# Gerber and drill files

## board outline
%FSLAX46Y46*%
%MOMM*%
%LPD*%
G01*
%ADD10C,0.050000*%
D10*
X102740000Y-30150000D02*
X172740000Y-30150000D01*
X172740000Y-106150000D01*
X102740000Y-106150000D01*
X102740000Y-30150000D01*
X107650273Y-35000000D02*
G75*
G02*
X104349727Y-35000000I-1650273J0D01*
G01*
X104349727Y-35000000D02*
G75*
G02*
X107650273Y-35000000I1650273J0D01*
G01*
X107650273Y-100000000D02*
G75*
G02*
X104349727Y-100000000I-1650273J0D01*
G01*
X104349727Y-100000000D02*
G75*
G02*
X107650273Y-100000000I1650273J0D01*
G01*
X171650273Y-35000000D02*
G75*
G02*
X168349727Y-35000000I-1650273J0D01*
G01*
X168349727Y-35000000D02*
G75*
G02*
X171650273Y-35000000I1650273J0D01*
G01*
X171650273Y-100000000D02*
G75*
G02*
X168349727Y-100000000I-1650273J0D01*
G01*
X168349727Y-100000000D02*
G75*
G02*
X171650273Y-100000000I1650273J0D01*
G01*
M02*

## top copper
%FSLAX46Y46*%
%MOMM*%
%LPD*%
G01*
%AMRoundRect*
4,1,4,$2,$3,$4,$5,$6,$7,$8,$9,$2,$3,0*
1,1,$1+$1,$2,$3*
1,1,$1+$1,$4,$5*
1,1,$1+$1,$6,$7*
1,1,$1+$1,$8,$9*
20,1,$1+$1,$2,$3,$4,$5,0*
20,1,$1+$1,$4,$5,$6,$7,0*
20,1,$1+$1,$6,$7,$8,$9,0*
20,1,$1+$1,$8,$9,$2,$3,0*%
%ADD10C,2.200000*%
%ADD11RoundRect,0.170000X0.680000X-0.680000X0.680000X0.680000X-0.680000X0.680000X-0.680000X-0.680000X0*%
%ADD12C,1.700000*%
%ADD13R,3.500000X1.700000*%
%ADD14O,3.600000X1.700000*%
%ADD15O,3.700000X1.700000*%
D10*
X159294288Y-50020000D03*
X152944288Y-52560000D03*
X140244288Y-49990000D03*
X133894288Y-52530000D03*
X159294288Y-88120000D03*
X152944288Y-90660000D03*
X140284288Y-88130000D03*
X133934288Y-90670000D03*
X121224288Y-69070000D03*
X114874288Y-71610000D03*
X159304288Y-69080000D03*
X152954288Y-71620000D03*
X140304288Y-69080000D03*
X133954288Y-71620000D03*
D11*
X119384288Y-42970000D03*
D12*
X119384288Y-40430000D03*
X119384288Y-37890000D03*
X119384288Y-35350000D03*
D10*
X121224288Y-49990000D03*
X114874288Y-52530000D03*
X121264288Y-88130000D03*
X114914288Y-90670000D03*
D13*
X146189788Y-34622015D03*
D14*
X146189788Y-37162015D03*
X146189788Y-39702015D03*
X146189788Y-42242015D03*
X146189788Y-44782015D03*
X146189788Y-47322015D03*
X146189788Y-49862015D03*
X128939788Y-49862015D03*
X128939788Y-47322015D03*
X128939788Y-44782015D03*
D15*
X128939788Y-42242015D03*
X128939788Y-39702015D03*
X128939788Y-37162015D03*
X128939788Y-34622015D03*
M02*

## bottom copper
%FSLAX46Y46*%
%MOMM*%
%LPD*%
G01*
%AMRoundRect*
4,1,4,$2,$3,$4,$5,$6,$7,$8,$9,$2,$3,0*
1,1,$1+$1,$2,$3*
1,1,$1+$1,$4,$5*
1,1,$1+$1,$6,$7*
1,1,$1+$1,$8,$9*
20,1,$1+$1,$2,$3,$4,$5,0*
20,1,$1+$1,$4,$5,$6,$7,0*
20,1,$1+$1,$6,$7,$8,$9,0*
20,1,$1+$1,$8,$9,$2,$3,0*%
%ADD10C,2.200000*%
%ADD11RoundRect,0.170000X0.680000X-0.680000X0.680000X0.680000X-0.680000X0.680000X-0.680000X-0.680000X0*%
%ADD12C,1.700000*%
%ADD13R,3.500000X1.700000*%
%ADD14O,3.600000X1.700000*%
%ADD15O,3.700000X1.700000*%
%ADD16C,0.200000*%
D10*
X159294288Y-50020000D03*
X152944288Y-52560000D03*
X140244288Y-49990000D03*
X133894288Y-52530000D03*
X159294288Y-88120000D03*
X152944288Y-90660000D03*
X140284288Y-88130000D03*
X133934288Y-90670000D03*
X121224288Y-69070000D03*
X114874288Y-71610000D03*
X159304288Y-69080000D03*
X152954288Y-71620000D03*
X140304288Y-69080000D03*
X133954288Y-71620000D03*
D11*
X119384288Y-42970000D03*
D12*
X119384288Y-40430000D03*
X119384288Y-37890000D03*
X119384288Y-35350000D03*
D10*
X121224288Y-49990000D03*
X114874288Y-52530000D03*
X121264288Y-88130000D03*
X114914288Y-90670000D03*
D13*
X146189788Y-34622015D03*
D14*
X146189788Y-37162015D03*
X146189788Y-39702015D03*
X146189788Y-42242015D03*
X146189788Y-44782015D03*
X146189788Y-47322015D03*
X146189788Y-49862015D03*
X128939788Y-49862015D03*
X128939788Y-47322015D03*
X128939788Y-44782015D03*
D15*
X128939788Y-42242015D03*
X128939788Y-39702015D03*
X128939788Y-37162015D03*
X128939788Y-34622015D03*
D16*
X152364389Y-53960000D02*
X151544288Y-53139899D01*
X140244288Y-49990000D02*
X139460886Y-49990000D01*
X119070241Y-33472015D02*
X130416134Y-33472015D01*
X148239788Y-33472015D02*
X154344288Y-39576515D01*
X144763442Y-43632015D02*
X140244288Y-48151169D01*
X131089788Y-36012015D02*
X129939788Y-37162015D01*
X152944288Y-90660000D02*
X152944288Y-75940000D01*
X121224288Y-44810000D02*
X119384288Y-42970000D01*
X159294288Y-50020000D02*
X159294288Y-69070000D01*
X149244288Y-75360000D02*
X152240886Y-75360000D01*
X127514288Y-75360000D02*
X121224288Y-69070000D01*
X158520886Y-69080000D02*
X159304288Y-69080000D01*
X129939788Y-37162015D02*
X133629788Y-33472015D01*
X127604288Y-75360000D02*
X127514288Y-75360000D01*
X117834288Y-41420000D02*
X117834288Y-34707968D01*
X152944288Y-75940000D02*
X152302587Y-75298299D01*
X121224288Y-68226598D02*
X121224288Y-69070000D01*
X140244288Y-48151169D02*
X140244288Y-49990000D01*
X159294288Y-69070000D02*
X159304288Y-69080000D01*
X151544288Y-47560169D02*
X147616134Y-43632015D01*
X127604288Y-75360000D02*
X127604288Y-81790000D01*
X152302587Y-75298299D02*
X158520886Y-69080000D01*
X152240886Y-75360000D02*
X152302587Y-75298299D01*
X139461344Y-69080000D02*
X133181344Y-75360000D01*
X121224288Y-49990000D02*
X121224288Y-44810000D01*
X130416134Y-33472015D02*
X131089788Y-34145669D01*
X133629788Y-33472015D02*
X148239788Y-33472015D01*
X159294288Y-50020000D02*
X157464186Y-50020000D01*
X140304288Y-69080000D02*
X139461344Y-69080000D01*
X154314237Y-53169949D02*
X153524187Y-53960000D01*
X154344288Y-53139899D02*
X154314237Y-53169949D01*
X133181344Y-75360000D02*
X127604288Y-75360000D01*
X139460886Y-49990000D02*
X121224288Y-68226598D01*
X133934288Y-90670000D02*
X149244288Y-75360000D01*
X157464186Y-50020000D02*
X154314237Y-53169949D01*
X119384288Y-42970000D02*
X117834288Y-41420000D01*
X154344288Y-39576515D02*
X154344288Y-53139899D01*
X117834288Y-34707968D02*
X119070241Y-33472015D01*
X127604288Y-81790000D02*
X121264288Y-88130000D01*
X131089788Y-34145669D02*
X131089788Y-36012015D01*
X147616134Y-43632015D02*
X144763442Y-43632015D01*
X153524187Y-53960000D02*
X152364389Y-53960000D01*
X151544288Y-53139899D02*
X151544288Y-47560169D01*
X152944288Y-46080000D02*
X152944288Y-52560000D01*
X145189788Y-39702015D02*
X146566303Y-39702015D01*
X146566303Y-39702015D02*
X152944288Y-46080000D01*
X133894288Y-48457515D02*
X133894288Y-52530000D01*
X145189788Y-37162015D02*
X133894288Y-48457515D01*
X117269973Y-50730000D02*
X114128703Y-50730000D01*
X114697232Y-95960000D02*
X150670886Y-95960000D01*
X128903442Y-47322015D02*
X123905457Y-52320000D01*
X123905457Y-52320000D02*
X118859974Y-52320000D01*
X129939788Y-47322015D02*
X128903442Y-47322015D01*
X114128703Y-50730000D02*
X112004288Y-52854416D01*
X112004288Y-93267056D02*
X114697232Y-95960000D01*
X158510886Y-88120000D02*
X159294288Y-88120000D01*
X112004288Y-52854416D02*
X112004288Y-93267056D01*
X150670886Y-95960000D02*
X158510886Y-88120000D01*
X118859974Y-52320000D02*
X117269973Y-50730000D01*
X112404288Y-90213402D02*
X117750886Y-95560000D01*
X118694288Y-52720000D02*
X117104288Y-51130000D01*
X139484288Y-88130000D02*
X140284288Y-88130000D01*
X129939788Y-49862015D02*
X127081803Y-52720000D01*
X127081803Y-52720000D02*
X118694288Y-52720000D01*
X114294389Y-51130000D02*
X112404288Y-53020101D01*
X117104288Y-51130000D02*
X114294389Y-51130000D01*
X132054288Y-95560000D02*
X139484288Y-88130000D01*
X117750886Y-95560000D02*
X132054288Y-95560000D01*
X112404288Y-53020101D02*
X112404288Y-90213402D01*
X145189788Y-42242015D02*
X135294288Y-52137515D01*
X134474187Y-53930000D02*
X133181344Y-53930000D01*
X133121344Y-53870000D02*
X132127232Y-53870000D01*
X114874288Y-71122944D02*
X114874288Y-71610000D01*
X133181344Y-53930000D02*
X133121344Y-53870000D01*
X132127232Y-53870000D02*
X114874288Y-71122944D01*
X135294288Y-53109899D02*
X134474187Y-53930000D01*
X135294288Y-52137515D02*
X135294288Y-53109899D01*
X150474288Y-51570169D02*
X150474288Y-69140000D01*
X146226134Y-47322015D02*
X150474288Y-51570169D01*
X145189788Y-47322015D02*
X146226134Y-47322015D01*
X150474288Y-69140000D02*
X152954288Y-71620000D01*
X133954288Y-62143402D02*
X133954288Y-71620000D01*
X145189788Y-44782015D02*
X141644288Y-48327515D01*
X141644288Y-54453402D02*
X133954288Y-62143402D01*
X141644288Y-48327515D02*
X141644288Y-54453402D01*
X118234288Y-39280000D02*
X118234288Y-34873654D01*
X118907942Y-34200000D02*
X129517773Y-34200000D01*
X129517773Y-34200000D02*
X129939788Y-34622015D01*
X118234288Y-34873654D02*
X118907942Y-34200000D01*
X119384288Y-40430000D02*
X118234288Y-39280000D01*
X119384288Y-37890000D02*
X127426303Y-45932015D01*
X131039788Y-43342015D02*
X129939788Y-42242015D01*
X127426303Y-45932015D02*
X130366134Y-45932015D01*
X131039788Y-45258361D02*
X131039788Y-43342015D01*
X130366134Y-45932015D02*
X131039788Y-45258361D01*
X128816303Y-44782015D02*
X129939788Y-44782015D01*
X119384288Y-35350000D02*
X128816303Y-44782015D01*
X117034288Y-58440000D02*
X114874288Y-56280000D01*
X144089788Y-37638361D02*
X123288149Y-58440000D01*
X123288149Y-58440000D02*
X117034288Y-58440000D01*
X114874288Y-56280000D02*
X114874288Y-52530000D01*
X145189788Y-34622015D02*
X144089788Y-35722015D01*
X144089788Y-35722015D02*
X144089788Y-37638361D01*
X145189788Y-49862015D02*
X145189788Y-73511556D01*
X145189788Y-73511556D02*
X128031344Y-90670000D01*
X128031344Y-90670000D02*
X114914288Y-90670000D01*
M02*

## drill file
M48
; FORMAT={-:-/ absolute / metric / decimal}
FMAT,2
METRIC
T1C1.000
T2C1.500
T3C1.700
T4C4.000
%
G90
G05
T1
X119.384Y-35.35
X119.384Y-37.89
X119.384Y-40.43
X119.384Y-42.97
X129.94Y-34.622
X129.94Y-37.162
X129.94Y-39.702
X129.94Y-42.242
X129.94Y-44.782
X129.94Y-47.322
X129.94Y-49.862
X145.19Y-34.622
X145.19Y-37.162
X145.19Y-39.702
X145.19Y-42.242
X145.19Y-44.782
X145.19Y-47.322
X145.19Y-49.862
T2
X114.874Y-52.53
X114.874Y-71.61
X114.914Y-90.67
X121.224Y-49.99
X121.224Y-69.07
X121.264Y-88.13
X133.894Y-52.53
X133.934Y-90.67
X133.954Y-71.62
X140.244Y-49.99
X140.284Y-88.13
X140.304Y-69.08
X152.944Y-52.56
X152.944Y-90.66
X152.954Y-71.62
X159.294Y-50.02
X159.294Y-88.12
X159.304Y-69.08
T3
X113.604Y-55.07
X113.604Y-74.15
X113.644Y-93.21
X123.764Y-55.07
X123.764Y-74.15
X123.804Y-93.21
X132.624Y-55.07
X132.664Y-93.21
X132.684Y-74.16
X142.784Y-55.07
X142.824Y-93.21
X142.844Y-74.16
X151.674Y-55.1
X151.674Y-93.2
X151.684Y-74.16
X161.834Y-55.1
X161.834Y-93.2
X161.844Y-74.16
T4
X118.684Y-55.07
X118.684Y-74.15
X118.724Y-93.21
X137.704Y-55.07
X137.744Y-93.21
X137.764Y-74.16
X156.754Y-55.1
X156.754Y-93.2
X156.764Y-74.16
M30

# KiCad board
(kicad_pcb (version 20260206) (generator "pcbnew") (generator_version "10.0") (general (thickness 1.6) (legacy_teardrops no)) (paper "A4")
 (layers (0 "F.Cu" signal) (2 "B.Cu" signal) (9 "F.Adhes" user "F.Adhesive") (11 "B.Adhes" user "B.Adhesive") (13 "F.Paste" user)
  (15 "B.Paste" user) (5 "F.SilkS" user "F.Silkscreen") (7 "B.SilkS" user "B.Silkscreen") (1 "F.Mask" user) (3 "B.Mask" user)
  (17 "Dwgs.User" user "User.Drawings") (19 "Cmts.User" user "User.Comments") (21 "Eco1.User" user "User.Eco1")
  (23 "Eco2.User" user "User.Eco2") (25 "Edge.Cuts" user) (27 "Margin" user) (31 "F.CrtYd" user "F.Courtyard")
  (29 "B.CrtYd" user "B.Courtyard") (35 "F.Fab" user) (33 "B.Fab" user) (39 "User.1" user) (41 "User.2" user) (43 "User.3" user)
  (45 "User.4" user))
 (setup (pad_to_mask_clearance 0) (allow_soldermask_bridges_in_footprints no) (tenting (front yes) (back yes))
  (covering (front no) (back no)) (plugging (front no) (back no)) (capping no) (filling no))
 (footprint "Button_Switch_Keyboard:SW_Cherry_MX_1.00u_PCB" (layer "F.Cu") (at 159.294288 50.02)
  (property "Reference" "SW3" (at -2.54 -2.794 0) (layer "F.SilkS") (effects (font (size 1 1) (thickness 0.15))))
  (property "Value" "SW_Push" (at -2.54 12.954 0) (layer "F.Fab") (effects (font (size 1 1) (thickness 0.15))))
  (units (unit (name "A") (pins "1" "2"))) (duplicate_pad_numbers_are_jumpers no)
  (pad "" np_thru_hole circle (at -7.62 5.08) (size 1.7 1.7) (drill 1.7) (layers "*.Cu" "*.Mask"))
  (pad "" np_thru_hole circle (at -2.54 5.08) (size 4 4) (drill 4) (layers "*.Cu" "*.Mask"))
  (pad "" np_thru_hole circle (at 2.54 5.08) (size 1.7 1.7) (drill 1.7) (layers "*.Cu" "*.Mask"))
  (pad "1" thru_hole circle (at 0 0) (size 2.2 2.2) (drill 1.5) (layers "*.Cu" "*.Mask") (remove_unused_layers no) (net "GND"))
  (pad "2" thru_hole circle (at -6.35 2.54) (size 2.2 2.2) (drill 1.5) (layers "*.Cu" "*.Mask") (remove_unused_layers no)
   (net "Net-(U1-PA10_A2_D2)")))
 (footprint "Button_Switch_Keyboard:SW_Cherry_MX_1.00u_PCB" (layer "F.Cu") (at 140.244288 49.99)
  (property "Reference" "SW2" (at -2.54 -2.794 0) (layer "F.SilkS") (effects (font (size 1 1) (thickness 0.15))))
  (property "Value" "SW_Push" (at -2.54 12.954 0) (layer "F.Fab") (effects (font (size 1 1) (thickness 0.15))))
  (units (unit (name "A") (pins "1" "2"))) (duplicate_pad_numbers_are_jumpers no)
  (pad "" np_thru_hole circle (at -7.62 5.08) (size 1.7 1.7) (drill 1.7) (layers "*.Cu" "*.Mask"))
  (pad "" np_thru_hole circle (at -2.54 5.08) (size 4 4) (drill 4) (layers "*.Cu" "*.Mask"))
  (pad "" np_thru_hole circle (at 2.54 5.08) (size 1.7 1.7) (drill 1.7) (layers "*.Cu" "*.Mask"))
  (pad "1" thru_hole circle (at 0 0) (size 2.2 2.2) (drill 1.5) (layers "*.Cu" "*.Mask") (remove_unused_layers no) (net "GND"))
  (pad "2" thru_hole circle (at -6.35 2.54) (size 2.2 2.2) (drill 1.5) (layers "*.Cu" "*.Mask") (remove_unused_layers no)
   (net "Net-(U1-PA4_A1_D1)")))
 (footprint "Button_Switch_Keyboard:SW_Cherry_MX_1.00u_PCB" (layer "F.Cu") (at 159.294288 88.12)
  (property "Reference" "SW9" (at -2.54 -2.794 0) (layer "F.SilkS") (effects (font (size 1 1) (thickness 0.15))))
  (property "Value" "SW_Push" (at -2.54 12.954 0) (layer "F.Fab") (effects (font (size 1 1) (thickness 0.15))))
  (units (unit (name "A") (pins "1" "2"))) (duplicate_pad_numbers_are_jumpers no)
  (pad "" np_thru_hole circle (at -7.62 5.08) (size 1.7 1.7) (drill 1.7) (layers "*.Cu" "*.Mask"))
  (pad "" np_thru_hole circle (at -2.54 5.08) (size 4 4) (drill 4) (layers "*.Cu" "*.Mask"))
  (pad "" np_thru_hole circle (at 2.54 5.08) (size 1.7 1.7) (drill 1.7) (layers "*.Cu" "*.Mask"))
  (pad "1" thru_hole circle (at 0 0) (size 2.2 2.2) (drill 1.5) (layers "*.Cu" "*.Mask") (remove_unused_layers no)
   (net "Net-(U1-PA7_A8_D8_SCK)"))
  (pad "2" thru_hole circle (at -6.35 2.54) (size 2.2 2.2) (drill 1.5) (layers "*.Cu" "*.Mask") (remove_unused_layers no) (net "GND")))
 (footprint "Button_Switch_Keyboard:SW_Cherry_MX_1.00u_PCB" (layer "F.Cu") (at 140.284288 88.13)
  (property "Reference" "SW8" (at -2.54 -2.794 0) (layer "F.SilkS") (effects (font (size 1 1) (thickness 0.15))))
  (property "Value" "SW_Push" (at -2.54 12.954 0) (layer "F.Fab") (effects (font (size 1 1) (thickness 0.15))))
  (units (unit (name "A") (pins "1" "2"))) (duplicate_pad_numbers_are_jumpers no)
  (pad "" np_thru_hole circle (at -7.62 5.08) (size 1.7 1.7) (drill 1.7) (layers "*.Cu" "*.Mask"))
  (pad "" np_thru_hole circle (at -2.54 5.08) (size 4 4) (drill 4) (layers "*.Cu" "*.Mask"))
  (pad "" np_thru_hole circle (at 2.54 5.08) (size 1.7 1.7) (drill 1.7) (layers "*.Cu" "*.Mask"))
  (pad "1" thru_hole circle (at 0 0) (size 2.2 2.2) (drill 1.5) (layers "*.Cu" "*.Mask") (remove_unused_layers no)
   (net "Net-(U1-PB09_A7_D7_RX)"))
  (pad "2" thru_hole circle (at -6.35 2.54) (size 2.2 2.2) (drill 1.5) (layers "*.Cu" "*.Mask") (remove_unused_layers no) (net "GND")))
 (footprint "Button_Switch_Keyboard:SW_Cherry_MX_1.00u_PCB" (layer "F.Cu") (at 121.224288 69.07)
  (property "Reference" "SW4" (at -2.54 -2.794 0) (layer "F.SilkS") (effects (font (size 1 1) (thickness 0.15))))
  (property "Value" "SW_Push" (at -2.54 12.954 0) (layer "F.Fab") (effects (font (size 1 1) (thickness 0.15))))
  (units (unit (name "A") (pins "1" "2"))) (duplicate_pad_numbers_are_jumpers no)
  (pad "" np_thru_hole circle (at -7.62 5.08) (size 1.7 1.7) (drill 1.7) (layers "*.Cu" "*.Mask"))
  (pad "" np_thru_hole circle (at -2.54 5.08) (size 4 4) (drill 4) (layers "*.Cu" "*.Mask"))
  (pad "" np_thru_hole circle (at 2.54 5.08) (size 1.7 1.7) (drill 1.7) (layers "*.Cu" "*.Mask"))
  (pad "1" thru_hole circle (at 0 0) (size 2.2 2.2) (drill 1.5) (layers "*.Cu" "*.Mask") (remove_unused_layers no) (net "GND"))
  (pad "2" thru_hole circle (at -6.35 2.54) (size 2.2 2.2) (drill 1.5) (layers "*.Cu" "*.Mask") (remove_unused_layers no)
   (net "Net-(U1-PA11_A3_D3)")))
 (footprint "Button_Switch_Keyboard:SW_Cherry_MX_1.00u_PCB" (layer "F.Cu") (at 159.304288 69.08)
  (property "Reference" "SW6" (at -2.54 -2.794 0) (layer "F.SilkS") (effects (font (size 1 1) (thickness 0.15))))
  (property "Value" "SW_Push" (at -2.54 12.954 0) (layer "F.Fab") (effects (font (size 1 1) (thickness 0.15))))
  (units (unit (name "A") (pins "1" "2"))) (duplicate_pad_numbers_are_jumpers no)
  (pad "" np_thru_hole circle (at -7.62 5.08) (size 1.7 1.7) (drill 1.7) (layers "*.Cu" "*.Mask"))
  (pad "" np_thru_hole circle (at -2.54 5.08) (size 4 4) (drill 4) (layers "*.Cu" "*.Mask"))
  (pad "" np_thru_hole circle (at 2.54 5.08) (size 1.7 1.7) (drill 1.7) (layers "*.Cu" "*.Mask"))
  (pad "1" thru_hole circle (at 0 0) (size 2.2 2.2) (drill 1.5) (layers "*.Cu" "*.Mask") (remove_unused_layers no) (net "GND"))
  (pad "2" thru_hole circle (at -6.35 2.54) (size 2.2 2.2) (drill 1.5) (layers "*.Cu" "*.Mask") (remove_unused_layers no)
   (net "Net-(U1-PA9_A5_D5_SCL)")))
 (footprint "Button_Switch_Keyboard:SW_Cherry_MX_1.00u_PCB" (layer "F.Cu") (at 140.304288 69.08)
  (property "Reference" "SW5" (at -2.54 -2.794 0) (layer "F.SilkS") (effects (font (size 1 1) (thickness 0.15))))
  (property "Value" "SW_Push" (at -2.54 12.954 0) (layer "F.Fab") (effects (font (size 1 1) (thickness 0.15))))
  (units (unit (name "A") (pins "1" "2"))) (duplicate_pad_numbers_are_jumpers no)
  (pad "" np_thru_hole circle (at -7.62 5.08) (size 1.7 1.7) (drill 1.7) (layers "*.Cu" "*.Mask"))
  (pad "" np_thru_hole circle (at -2.54 5.08) (size 4 4) (drill 4) (layers "*.Cu" "*.Mask"))
  (pad "" np_thru_hole circle (at 2.54 5.08) (size 1.7 1.7) (drill 1.7) (layers "*.Cu" "*.Mask"))
  (pad "1" thru_hole circle (at 0 0) (size 2.2 2.2) (drill 1.5) (layers "*.Cu" "*.Mask") (remove_unused_layers no) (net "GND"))
  (pad "2" thru_hole circle (at -6.35 2.54) (size 2.2 2.2) (drill 1.5) (layers "*.Cu" "*.Mask") (remove_unused_layers no)
   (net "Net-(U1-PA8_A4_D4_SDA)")))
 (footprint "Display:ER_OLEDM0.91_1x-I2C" (layer "F.Cu") (at 119.384288 42.97 90)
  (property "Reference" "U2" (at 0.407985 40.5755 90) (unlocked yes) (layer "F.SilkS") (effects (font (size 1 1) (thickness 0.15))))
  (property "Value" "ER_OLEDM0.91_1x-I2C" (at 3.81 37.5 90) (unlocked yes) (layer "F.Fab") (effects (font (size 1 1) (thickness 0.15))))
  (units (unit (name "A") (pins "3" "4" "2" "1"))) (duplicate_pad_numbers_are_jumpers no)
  (pad "1" thru_hole roundrect (at 0 0 90) (size 1.7 1.7) (drill 1) (layers "*.Cu" "*.Mask") (remove_unused_layers no)
   (roundrect_rratio 0.1) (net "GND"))
  (pad "2" thru_hole circle (at 2.54 0 90) (size 1.7 1.7) (drill 1) (layers "*.Cu" "*.Mask") (remove_unused_layers no) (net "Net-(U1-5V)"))
  (pad "3" thru_hole circle (at 5.08 0 90) (size 1.7 1.7) (drill 1) (layers "*.Cu" "*.Mask") (remove_unused_layers no)
   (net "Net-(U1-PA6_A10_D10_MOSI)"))
  (pad "4" thru_hole circle (at 7.62 0 90) (size 1.7 1.7) (drill 1) (layers "*.Cu" "*.Mask") (remove_unused_layers no)
   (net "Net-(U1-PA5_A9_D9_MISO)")))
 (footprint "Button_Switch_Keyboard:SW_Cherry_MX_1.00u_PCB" (layer "F.Cu") (at 121.224288 49.99)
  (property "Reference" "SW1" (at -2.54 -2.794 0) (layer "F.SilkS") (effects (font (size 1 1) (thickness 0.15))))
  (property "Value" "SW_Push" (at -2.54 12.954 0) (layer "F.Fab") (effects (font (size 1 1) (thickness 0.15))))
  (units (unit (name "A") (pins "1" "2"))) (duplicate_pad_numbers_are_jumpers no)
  (pad "" np_thru_hole circle (at -7.62 5.08) (size 1.7 1.7) (drill 1.7) (layers "*.Cu" "*.Mask"))
  (pad "" np_thru_hole circle (at -2.54 5.08) (size 4 4) (drill 4) (layers "*.Cu" "*.Mask"))
  (pad "" np_thru_hole circle (at 2.54 5.08) (size 1.7 1.7) (drill 1.7) (layers "*.Cu" "*.Mask"))
  (pad "1" thru_hole circle (at 0 0) (size 2.2 2.2) (drill 1.5) (layers "*.Cu" "*.Mask") (remove_unused_layers no) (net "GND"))
  (pad "2" thru_hole circle (at -6.35 2.54) (size 2.2 2.2) (drill 1.5) (layers "*.Cu" "*.Mask") (remove_unused_layers no)
   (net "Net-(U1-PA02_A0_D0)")))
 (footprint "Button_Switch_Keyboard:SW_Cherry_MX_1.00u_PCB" (layer "F.Cu") (at 121.264288 88.13)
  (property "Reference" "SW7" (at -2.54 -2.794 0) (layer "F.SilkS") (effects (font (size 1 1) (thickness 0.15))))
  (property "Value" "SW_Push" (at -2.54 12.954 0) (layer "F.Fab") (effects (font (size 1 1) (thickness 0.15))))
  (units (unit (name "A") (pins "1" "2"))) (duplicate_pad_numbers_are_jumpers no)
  (pad "" np_thru_hole circle (at -7.62 5.08) (size 1.7 1.7) (drill 1.7) (layers "*.Cu" "*.Mask"))
  (pad "" np_thru_hole circle (at -2.54 5.08) (size 4 4) (drill 4) (layers "*.Cu" "*.Mask"))
  (pad "" np_thru_hole circle (at 2.54 5.08) (size 1.7 1.7) (drill 1.7) (layers "*.Cu" "*.Mask"))
  (pad "1" thru_hole circle (at 0 0) (size 2.2 2.2) (drill 1.5) (layers "*.Cu" "*.Mask") (remove_unused_layers no) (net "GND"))
  (pad "2" thru_hole circle (at -6.35 2.54) (size 2.2 2.2) (drill 1.5) (layers "*.Cu" "*.Mask") (remove_unused_layers no)
   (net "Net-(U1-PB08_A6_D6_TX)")))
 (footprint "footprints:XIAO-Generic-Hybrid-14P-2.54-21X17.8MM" (layer "B.Cu") (at 137.564788 42.242015 180)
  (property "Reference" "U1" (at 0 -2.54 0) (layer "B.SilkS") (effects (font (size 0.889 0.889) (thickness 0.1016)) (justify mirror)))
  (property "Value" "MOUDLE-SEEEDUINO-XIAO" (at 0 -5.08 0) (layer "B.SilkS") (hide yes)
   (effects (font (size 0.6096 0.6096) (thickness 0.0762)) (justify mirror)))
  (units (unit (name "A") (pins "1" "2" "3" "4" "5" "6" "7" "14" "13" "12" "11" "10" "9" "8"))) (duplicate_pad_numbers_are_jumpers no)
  (pad "1" thru_hole rect (at -7.625 7.62 180) (size 3.5 1.7) (drill 1 (offset -1 0)) (layers "*.Cu" "*.Mask") (remove_unused_layers no)
   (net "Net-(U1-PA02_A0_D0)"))
  (pad "2" thru_hole oval (at -7.625 5.08 180) (size 3.6 1.7) (drill 1 (offset -1 0)) (layers "*.Cu" "*.Mask") (remove_unused_layers no)
   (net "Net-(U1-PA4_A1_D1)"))
  (pad "3" thru_hole oval (at -7.625 2.54 180) (size 3.6 1.7) (drill 1 (offset -1 0)) (layers "*.Cu" "*.Mask") (remove_unused_layers no)
   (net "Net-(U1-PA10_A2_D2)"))
  (pad "4" thru_hole oval (at -7.625 0 180) (size 3.6 1.7) (drill 1 (offset -1 0)) (layers "*.Cu" "*.Mask") (remove_unused_layers no)
   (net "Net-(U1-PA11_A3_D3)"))
  (pad "5" thru_hole oval (at -7.625 -2.54 180) (size 3.6 1.7) (drill 1 (offset -1 0)) (layers "*.Cu" "*.Mask") (remove_unused_layers no)
   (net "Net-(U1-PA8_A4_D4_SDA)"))
  (pad "6" thru_hole oval (at -7.625 -5.08) (size 3.6 1.7) (drill 1 (offset 1 0)) (layers "*.Cu" "*.Mask") (remove_unused_layers no)
   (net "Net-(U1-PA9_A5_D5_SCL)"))
  (pad "7" thru_hole oval (at -7.625 -7.62 180) (size 3.6 1.7) (drill 1 (offset -1 0)) (layers "*.Cu" "*.Mask") (remove_unused_layers no)
   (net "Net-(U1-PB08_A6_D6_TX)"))
  (pad "8" thru_hole oval (at 7.625 -7.62 180) (size 3.6 1.7) (drill 1 (offset 1 0)) (layers "*.Cu" "*.Mask") (remove_unused_layers no)
   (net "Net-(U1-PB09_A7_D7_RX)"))
  (pad "9" thru_hole oval (at 7.625 -5.08 180) (size 3.6 1.7) (drill 1 (offset 1 0)) (layers "*.Cu" "*.Mask") (remove_unused_layers no)
   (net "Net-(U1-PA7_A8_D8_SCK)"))
  (pad "10" thru_hole oval (at 7.625 -2.54 180) (size 3.6 1.7) (drill 1 (offset 1 0)) (layers "*.Cu" "*.Mask") (remove_unused_layers no)
   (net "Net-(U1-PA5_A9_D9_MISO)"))
  (pad "11" thru_hole oval (at 7.625 0 180) (size 3.7 1.7) (drill 1 (offset 1 0)) (layers "*.Cu" "*.Mask") (remove_unused_layers no)
   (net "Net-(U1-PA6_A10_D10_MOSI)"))
  (pad "12" thru_hole oval (at 7.625 2.54 180) (size 3.7 1.7) (drill 1 (offset 1 0)) (layers "*.Cu" "*.Mask") (remove_unused_layers no)
   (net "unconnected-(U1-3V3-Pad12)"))
  (pad "13" thru_hole oval (at 7.625 5.08 180) (size 3.7 1.7) (drill 1 (offset 1 0)) (layers "*.Cu" "*.Mask") (remove_unused_layers no)
   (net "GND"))
  (pad "14" thru_hole oval (at 7.625 7.62 180) (size 3.7 1.7) (drill 1 (offset 1 0)) (layers "*.Cu" "*.Mask") (remove_unused_layers no)
   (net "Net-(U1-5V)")))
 (gr_rect (start 102.74 30.15) (end 172.74 106.15) (stroke (width 0.05) (type solid)) (fill no) (layer "Edge.Cuts"))
 (gr_circle (center 106 35) (end 107.650273 35) (stroke (width 0.05) (type solid)) (fill no) (layer "Edge.Cuts"))
 (gr_circle (center 106 100) (end 107.650273 100) (stroke (width 0.05) (type solid)) (fill no) (layer "Edge.Cuts"))
 (gr_circle (center 170 35) (end 171.650273 35) (stroke (width 0.05) (type solid)) (fill no) (layer "Edge.Cuts"))
 (gr_circle (center 170 100) (end 171.650273 100) (stroke (width 0.05) (type solid)) (fill no) (layer "Edge.Cuts"))
 (segment (start 152.364389 53.96) (end 151.544288 53.139899) (width 0.2) (layer "B.Cu") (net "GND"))
 (segment (start 140.244288 49.99) (end 139.460886 49.99) (width 0.2) (layer "B.Cu") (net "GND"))
 (segment (start 119.070241 33.472015) (end 130.416134 33.472015) (width 0.2) (layer "B.Cu") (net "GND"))
 (segment (start 148.239788 33.472015) (end 154.344288 39.576515) (width 0.2) (layer "B.Cu") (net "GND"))
 (segment (start 144.763442 43.632015) (end 140.244288 48.151169) (width 0.2) (layer "B.Cu") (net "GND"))
 (segment (start 131.089788 36.012015) (end 129.939788 37.162015) (width 0.2) (layer "B.Cu") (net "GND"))
 (segment (start 152.944288 90.66) (end 152.944288 75.94) (width 0.2) (layer "B.Cu") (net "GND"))
 (segment (start 121.224288 44.81) (end 119.384288 42.97) (width 0.2) (layer "B.Cu") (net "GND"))
 (segment (start 159.294288 50.02) (end 159.294288 69.07) (width 0.2) (layer "B.Cu") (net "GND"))
 (segment (start 149.244288 75.36) (end 152.240886 75.36) (width 0.2) (layer "B.Cu") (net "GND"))
 (segment (start 127.514288 75.36) (end 121.224288 69.07) (width 0.2) (layer "B.Cu") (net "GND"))
 (segment (start 158.520886 69.08) (end 159.304288 69.08) (width 0.2) (layer "B.Cu") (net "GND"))
 (segment (start 129.939788 37.162015) (end 133.629788 33.472015) (width 0.2) (layer "B.Cu") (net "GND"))
 (segment (start 127.604288 75.36) (end 127.514288 75.36) (width 0.2) (layer "B.Cu") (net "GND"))
 (segment (start 117.834288 41.42) (end 117.834288 34.707968) (width 0.2) (layer "B.Cu") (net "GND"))
 (segment (start 152.944288 75.94) (end 152.302587 75.298299) (width 0.2) (layer "B.Cu") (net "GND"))
 (segment (start 121.224288 68.226598) (end 121.224288 69.07) (width 0.2) (layer "B.Cu") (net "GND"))
 (segment (start 140.244288 48.151169) (end 140.244288 49.99) (width 0.2) (layer "B.Cu") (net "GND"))
 (segment (start 159.294288 69.07) (end 159.304288 69.08) (width 0.2) (layer "B.Cu") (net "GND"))
 (segment (start 151.544288 47.560169) (end 147.616134 43.632015) (width 0.2) (layer "B.Cu") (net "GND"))
 (segment (start 127.604288 75.36) (end 127.604288 81.79) (width 0.2) (layer "B.Cu") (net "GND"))
 (segment (start 152.302587 75.298299) (end 158.520886 69.08) (width 0.2) (layer "B.Cu") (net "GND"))
 (segment (start 152.240886 75.36) (end 152.302587 75.298299) (width 0.2) (layer "B.Cu") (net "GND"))
 (segment (start 139.461344 69.08) (end 133.181344 75.36) (width 0.2) (layer "B.Cu") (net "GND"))
 (segment (start 121.224288 49.99) (end 121.224288 44.81) (width 0.2) (layer "B.Cu") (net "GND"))
 (segment (start 130.416134 33.472015) (end 131.089788 34.145669) (width 0.2) (layer "B.Cu") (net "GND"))
 (segment (start 133.629788 33.472015) (end 148.239788 33.472015) (width 0.2) (layer "B.Cu") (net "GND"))
 (segment (start 159.294288 50.02) (end 157.464186 50.02) (width 0.2) (layer "B.Cu") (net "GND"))
 (segment (start 140.304288 69.08) (end 139.461344 69.08) (width 0.2) (layer "B.Cu") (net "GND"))
 (segment (start 154.314237 53.169949) (end 153.524187 53.96) (width 0.2) (layer "B.Cu") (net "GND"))
 (segment (start 154.344288 53.139899) (end 154.314237 53.169949) (width 0.2) (layer "B.Cu") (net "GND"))
 (segment (start 133.181344 75.36) (end 127.604288 75.36) (width 0.2) (layer "B.Cu") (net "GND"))
 (segment (start 139.460886 49.99) (end 121.224288 68.226598) (width 0.2) (layer "B.Cu") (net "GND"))
 (segment (start 133.934288 90.67) (end 149.244288 75.36) (width 0.2) (layer "B.Cu") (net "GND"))
 (segment (start 157.464186 50.02) (end 154.314237 53.169949) (width 0.2) (layer "B.Cu") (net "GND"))
 (segment (start 119.384288 42.97) (end 117.834288 41.42) (width 0.2) (layer "B.Cu") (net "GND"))
 (segment (start 154.344288 39.576515) (end 154.344288 53.139899) (width 0.2) (layer "B.Cu") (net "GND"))
 (segment (start 117.834288 34.707968) (end 119.070241 33.472015) (width 0.2) (layer "B.Cu") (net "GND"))
 (segment (start 127.604288 81.79) (end 121.264288 88.13) (width 0.2) (layer "B.Cu") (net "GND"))
 (segment (start 131.089788 34.145669) (end 131.089788 36.012015) (width 0.2) (layer "B.Cu") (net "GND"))
 (segment (start 147.616134 43.632015) (end 144.763442 43.632015) (width 0.2) (layer "B.Cu") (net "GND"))
 (segment (start 153.524187 53.96) (end 152.364389 53.96) (width 0.2) (layer "B.Cu") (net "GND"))
 (segment (start 151.544288 53.139899) (end 151.544288 47.560169) (width 0.2) (layer "B.Cu") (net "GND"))
 (segment (start 152.944288 46.08) (end 152.944288 52.56) (width 0.2) (layer "B.Cu") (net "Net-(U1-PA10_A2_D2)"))
 (segment (start 145.189788 39.702015) (end 146.566303 39.702015) (width 0.2) (layer "B.Cu") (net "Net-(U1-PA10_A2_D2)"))
 (segment (start 146.566303 39.702015) (end 152.944288 46.08) (width 0.2) (layer "B.Cu") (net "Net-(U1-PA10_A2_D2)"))
 (segment (start 133.894288 48.457515) (end 133.894288 52.53) (width 0.2) (layer "B.Cu") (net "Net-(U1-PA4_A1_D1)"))
 (segment (start 145.189788 37.162015) (end 133.894288 48.457515) (width 0.2) (layer "B.Cu") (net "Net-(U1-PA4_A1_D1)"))
 (segment (start 117.269973 50.73) (end 114.128703 50.73) (width 0.2) (layer "B.Cu") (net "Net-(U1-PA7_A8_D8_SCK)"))
 (segment (start 114.697232 95.96) (end 150.670886 95.96) (width 0.2) (layer "B.Cu") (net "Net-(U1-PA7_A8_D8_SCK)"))
 (segment (start 128.903442 47.322015) (end 123.905457 52.32) (width 0.2) (layer "B.Cu") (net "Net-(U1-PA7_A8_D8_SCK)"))
 (segment (start 123.905457 52.32) (end 118.859974 52.32) (width 0.2) (layer "B.Cu") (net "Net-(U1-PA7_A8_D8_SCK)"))
 (segment (start 129.939788 47.322015) (end 128.903442 47.322015) (width 0.2) (layer "B.Cu") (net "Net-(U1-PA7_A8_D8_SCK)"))
 (segment (start 114.128703 50.73) (end 112.004288 52.854416) (width 0.2) (layer "B.Cu") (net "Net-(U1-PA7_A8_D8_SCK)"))
 (segment (start 112.004288 93.267056) (end 114.697232 95.96) (width 0.2) (layer "B.Cu") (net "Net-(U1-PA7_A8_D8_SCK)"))
 (segment (start 158.510886 88.12) (end 159.294288 88.12) (width 0.2) (layer "B.Cu") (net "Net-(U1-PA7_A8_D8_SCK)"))
 (segment (start 112.004288 52.854416) (end 112.004288 93.267056) (width 0.2) (layer "B.Cu") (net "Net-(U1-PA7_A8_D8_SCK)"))
 (segment (start 150.670886 95.96) (end 158.510886 88.12) (width 0.2) (layer "B.Cu") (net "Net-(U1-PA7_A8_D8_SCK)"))
 (segment (start 118.859974 52.32) (end 117.269973 50.73) (width 0.2) (layer "B.Cu") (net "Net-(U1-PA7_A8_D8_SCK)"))
 (segment (start 112.404288 90.213402) (end 117.750886 95.56) (width 0.2) (layer "B.Cu") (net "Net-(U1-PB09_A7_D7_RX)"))
 (segment (start 118.694288 52.72) (end 117.104288 51.13) (width 0.2) (layer "B.Cu") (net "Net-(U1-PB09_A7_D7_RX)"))
 (segment (start 139.484288 88.13) (end 140.284288 88.13) (width 0.2) (layer "B.Cu") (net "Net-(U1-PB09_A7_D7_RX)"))
 (segment (start 129.939788 49.862015) (end 127.081803 52.72) (width 0.2) (layer "B.Cu") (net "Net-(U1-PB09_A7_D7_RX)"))
 (segment (start 127.081803 52.72) (end 118.694288 52.72) (width 0.2) (layer "B.Cu") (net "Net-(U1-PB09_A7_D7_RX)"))
 (segment (start 114.294389 51.13) (end 112.404288 53.020101) (width 0.2) (layer "B.Cu") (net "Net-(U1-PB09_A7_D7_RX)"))
 (segment (start 117.104288 51.13) (end 114.294389 51.13) (width 0.2) (layer "B.Cu") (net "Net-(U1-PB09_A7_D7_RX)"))
 (segment (start 132.054288 95.56) (end 139.484288 88.13) (width 0.2) (layer "B.Cu") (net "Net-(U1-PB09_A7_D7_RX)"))
 (segment (start 117.750886 95.56) (end 132.054288 95.56) (width 0.2) (layer "B.Cu") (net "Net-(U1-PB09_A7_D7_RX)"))
 (segment (start 112.404288 53.020101) (end 112.404288 90.213402) (width 0.2) (layer "B.Cu") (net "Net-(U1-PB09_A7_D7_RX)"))
 (segment (start 145.189788 42.242015) (end 135.294288 52.137515) (width 0.2) (layer "B.Cu") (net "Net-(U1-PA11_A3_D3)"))
 (segment (start 134.474187 53.93) (end 133.181344 53.93) (width 0.2) (layer "B.Cu") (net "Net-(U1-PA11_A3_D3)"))
 (segment (start 133.121344 53.87) (end 132.127232 53.87) (width 0.2) (layer "B.Cu") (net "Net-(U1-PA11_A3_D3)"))
 (segment (start 114.874288 71.122944) (end 114.874288 71.61) (width 0.2) (layer "B.Cu") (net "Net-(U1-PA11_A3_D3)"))
 (segment (start 133.181344 53.93) (end 133.121344 53.87) (width 0.2) (layer "B.Cu") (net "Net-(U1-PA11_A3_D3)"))
 (segment (start 132.127232 53.87) (end 114.874288 71.122944) (width 0.2) (layer "B.Cu") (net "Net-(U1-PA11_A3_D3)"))
 (segment (start 135.294288 53.109899) (end 134.474187 53.93) (width 0.2) (layer "B.Cu") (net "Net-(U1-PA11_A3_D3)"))
 (segment (start 135.294288 52.137515) (end 135.294288 53.109899) (width 0.2) (layer "B.Cu") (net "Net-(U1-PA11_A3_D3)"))
 (segment (start 150.474288 51.570169) (end 150.474288 69.14) (width 0.2) (layer "B.Cu") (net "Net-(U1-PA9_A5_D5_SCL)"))
 (segment (start 146.226134 47.322015) (end 150.474288 51.570169) (width 0.2) (layer "B.Cu") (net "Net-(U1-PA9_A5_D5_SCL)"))
 (segment (start 145.189788 47.322015) (end 146.226134 47.322015) (width 0.2) (layer "B.Cu") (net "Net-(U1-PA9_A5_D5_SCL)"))
 (segment (start 150.474288 69.14) (end 152.954288 71.62) (width 0.2) (layer "B.Cu") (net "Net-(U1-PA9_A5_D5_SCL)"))
 (segment (start 133.954288 62.143402) (end 133.954288 71.62) (width 0.2) (layer "B.Cu") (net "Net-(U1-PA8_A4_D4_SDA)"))
 (segment (start 145.189788 44.782015) (end 141.644288 48.327515) (width 0.2) (layer "B.Cu") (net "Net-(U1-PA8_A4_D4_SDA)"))
 (segment (start 141.644288 54.453402) (end 133.954288 62.143402) (width 0.2) (layer "B.Cu") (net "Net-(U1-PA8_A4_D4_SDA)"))
 (segment (start 141.644288 48.327515) (end 141.644288 54.453402) (width 0.2) (layer "B.Cu") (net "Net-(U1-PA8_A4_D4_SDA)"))
 (segment (start 118.234288 39.28) (end 118.234288 34.873654) (width 0.2) (layer "B.Cu") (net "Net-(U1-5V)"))
 (segment (start 118.907942 34.2) (end 129.517773 34.2) (width 0.2) (layer "B.Cu") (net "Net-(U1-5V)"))
 (segment (start 129.517773 34.2) (end 129.939788 34.622015) (width 0.2) (layer "B.Cu") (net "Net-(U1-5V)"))
 (segment (start 118.234288 34.873654) (end 118.907942 34.2) (width 0.2) (layer "B.Cu") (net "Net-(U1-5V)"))
 (segment (start 119.384288 40.43) (end 118.234288 39.28) (width 0.2) (layer "B.Cu") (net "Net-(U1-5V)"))
 (segment (start 119.384288 37.89) (end 127.426303 45.932015) (width 0.2) (layer "B.Cu") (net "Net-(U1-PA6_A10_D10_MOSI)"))
 (segment (start 131.039788 43.342015) (end 129.939788 42.242015) (width 0.2) (layer "B.Cu") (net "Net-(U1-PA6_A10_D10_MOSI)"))
 (segment (start 127.426303 45.932015) (end 130.366134 45.932015) (width 0.2) (layer "B.Cu") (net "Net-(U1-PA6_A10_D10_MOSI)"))
 (segment (start 131.039788 45.258361) (end 131.039788 43.342015) (width 0.2) (layer "B.Cu") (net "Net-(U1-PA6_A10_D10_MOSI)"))
 (segment (start 130.366134 45.932015) (end 131.039788 45.258361) (width 0.2) (layer "B.Cu") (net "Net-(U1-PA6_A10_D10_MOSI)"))
 (segment (start 128.816303 44.782015) (end 129.939788 44.782015) (width 0.2) (layer "B.Cu") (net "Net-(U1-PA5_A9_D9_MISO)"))
 (segment (start 119.384288 35.35) (end 128.816303 44.782015) (width 0.2) (layer "B.Cu") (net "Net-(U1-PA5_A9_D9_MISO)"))
 (segment (start 117.034288 58.44) (end 114.874288 56.28) (width 0.2) (layer "B.Cu") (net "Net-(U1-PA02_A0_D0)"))
 (segment (start 144.089788 37.638361) (end 123.288149 58.44) (width 0.2) (layer "B.Cu") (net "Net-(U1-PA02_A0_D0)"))
 (segment (start 123.288149 58.44) (end 117.034288 58.44) (width 0.2) (layer "B.Cu") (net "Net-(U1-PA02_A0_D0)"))
 (segment (start 114.874288 56.28) (end 114.874288 52.53) (width 0.2) (layer "B.Cu") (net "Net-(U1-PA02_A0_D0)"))
 (segment (start 145.189788 34.622015) (end 144.089788 35.722015) (width 0.2) (layer "B.Cu") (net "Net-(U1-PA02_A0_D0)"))
 (segment (start 144.089788 35.722015) (end 144.089788 37.638361) (width 0.2) (layer "B.Cu") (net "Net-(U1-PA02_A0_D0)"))
 (segment (start 145.189788 49.862015) (end 145.189788 73.511556) (width 0.2) (layer "B.Cu") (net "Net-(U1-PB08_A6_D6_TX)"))
 (segment (start 145.189788 73.511556) (end 128.031344 90.67) (width 0.2) (layer "B.Cu") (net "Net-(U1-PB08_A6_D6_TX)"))
 (segment (start 128.031344 90.67) (end 114.914288 90.67) (width 0.2) (layer "B.Cu") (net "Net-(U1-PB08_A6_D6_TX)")))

